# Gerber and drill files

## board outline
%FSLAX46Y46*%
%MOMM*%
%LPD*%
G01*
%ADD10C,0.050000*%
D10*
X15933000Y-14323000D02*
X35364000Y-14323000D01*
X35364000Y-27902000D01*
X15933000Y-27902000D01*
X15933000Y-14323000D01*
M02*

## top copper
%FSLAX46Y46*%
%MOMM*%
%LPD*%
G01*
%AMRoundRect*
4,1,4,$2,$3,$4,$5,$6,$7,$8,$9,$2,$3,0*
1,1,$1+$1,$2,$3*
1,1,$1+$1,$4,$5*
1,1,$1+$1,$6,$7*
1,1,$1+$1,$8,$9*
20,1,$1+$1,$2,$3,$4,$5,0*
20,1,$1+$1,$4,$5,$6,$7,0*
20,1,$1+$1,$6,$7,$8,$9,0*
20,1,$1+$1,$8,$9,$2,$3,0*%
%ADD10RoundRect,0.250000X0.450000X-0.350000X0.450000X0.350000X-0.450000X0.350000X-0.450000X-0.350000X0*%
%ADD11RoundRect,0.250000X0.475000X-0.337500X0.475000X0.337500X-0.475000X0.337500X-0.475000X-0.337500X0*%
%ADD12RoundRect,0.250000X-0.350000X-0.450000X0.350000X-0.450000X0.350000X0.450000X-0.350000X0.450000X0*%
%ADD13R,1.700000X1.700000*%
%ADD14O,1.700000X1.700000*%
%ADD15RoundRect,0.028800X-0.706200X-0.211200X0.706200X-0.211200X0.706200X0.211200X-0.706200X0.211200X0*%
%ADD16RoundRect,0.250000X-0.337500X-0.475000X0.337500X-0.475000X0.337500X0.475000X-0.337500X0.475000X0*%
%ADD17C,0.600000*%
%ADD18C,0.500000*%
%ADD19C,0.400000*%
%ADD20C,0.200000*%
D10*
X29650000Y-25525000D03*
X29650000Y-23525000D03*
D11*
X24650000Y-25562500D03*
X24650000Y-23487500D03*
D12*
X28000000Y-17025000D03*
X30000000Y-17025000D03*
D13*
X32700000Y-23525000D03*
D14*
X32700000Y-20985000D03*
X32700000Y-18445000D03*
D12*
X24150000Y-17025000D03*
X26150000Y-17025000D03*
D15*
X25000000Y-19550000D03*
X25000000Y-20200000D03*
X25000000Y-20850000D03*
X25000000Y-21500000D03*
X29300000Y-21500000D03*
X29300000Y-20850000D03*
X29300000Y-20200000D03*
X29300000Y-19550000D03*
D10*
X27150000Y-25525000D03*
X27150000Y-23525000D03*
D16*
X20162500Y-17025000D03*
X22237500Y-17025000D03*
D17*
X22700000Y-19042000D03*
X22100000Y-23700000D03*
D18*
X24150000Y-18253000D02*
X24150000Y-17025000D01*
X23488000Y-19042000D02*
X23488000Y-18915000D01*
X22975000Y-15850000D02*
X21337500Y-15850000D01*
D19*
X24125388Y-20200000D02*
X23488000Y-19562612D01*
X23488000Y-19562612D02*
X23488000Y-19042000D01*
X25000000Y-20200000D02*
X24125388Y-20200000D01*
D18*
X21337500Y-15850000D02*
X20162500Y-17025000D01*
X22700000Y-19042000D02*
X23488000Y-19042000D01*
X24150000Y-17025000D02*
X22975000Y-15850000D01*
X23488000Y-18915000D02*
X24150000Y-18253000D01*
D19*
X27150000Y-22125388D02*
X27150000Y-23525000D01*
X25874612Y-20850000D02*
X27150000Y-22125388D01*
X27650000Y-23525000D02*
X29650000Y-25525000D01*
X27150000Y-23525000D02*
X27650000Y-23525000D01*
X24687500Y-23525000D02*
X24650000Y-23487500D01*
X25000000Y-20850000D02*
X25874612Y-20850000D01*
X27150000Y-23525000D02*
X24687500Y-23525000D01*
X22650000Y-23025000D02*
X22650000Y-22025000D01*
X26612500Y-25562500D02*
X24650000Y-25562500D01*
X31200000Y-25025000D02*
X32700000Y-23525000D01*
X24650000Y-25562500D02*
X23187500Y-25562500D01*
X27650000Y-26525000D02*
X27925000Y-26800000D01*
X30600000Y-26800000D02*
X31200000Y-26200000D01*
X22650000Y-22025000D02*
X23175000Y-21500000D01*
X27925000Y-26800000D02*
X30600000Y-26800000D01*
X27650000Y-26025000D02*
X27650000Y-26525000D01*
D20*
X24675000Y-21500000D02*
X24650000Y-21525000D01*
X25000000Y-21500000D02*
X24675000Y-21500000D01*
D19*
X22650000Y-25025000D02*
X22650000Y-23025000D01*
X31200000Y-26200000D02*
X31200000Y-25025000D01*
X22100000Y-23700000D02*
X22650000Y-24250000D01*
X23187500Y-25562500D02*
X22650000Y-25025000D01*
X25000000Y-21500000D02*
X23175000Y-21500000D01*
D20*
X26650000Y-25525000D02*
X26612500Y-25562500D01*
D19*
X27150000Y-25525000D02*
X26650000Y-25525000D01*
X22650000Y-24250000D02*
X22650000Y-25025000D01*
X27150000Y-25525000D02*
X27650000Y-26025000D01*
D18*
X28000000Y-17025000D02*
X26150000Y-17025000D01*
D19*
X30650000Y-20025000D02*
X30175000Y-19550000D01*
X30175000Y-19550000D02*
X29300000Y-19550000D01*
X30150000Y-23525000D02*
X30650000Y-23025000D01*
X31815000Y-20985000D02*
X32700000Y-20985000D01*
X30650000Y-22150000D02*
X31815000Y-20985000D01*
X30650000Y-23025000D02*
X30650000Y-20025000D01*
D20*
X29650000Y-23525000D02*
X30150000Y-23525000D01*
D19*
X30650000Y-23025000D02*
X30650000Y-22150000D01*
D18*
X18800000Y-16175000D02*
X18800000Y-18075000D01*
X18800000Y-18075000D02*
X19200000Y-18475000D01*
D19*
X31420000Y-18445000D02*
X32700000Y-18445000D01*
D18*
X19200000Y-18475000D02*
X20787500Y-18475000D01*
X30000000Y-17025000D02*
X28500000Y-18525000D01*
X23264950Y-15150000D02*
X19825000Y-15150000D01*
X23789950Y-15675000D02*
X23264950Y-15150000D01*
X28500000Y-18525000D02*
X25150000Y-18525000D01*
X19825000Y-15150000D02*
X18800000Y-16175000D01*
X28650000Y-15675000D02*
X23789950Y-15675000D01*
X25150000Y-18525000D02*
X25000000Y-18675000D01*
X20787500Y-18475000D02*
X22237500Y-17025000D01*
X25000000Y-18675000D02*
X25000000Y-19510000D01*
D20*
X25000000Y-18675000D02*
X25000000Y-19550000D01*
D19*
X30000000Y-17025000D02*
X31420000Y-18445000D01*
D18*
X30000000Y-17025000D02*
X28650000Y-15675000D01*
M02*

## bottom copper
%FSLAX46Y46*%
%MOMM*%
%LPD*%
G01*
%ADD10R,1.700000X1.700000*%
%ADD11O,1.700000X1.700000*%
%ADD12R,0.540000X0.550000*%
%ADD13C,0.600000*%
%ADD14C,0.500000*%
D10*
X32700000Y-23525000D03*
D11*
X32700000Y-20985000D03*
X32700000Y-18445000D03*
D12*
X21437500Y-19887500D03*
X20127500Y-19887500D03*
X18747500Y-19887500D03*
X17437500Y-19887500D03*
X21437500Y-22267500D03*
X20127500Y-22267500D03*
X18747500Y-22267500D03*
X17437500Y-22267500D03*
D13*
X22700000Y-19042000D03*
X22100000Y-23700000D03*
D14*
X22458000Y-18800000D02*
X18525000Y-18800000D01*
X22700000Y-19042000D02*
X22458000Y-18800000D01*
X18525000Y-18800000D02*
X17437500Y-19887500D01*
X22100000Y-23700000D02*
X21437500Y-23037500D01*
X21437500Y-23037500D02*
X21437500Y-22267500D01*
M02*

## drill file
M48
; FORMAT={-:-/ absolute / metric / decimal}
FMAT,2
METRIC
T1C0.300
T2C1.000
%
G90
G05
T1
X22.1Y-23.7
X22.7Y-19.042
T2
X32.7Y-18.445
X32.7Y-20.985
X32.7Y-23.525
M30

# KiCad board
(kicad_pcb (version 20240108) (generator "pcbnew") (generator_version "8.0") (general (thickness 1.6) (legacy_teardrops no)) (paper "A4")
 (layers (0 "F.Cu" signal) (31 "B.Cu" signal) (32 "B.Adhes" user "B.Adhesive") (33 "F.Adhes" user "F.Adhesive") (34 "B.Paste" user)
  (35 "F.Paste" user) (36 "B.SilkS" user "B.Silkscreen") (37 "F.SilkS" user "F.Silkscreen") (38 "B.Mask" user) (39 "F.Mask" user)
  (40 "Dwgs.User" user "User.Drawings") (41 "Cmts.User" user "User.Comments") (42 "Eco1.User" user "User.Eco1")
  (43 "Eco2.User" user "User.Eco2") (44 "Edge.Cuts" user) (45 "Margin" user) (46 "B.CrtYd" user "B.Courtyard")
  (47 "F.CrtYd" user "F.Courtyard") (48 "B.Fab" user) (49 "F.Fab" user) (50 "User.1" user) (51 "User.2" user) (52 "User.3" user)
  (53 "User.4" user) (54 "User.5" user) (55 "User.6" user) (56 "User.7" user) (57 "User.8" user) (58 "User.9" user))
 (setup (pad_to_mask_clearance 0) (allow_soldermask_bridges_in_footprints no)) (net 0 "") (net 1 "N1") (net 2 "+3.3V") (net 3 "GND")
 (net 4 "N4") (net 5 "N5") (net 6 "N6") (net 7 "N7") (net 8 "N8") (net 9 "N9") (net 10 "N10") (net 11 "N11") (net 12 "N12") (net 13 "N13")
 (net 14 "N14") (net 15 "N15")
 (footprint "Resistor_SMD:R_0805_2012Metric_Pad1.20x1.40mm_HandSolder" (layer "F.Cu") (at 29.65 24.525 90)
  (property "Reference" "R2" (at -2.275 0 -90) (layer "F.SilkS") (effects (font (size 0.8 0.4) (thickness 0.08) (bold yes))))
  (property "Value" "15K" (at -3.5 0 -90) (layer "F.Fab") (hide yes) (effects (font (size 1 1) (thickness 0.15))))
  (pad "1" smd roundrect (at -1 0 90) (size 1.2 1.4) (layers "F.Cu" "F.Paste" "F.Mask") (roundrect_rratio 0.208333) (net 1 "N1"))
  (pad "2" smd roundrect (at 1 0 90) (size 1.2 1.4) (layers "F.Cu" "F.Paste" "F.Mask") (roundrect_rratio 0.208333) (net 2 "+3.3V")))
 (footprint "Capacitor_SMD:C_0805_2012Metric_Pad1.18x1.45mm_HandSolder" (layer "F.Cu") (at 24.65 24.525 90)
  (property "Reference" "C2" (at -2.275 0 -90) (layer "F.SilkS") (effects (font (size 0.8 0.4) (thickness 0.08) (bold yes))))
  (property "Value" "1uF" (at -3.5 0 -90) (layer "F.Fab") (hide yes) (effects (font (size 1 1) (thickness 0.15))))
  (pad "1" smd roundrect (at -1.0375 0 90) (size 1.175 1.45) (layers "F.Cu" "F.Paste" "F.Mask") (roundrect_rratio 0.212766) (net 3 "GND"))
  (pad "2" smd roundrect (at 1.0375 0 90) (size 1.175 1.45) (layers "F.Cu" "F.Paste" "F.Mask") (roundrect_rratio 0.212766) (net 1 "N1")))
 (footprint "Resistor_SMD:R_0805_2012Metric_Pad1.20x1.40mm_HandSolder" (layer "F.Cu") (at 29 17.025)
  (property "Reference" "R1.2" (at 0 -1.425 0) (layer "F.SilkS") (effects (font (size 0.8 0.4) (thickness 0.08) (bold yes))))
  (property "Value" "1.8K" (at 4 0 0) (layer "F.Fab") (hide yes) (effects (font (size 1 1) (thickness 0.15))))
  (pad "1" smd roundrect (at -1 0) (size 1.2 1.4) (layers "F.Cu" "F.Paste" "F.Mask") (roundrect_rratio 0.208333) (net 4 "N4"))
  (pad "2" smd roundrect (at 1 0) (size 1.2 1.4) (layers "F.Cu" "F.Paste" "F.Mask") (roundrect_rratio 0.208333) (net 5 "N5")))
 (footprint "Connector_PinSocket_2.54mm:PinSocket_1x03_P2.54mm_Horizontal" (layer "F.Cu") (at 32.7 23.525 180)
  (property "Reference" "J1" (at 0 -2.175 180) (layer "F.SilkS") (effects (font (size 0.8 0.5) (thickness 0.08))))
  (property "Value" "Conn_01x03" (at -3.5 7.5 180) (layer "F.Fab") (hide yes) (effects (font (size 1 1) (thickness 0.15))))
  (pad "1" thru_hole rect (at 0 0 180) (size 1.7 1.7) (drill 1) (layers "*.Cu" "*.Mask") (remove_unused_layers no) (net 3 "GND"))
  (pad "2" thru_hole oval (at 0 2.54 180) (size 1.7 1.7) (drill 1) (layers "*.Cu" "*.Mask") (remove_unused_layers no) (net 2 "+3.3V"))
  (pad "3" thru_hole oval (at 0 5.08 180) (size 1.7 1.7) (drill 1) (layers "*.Cu" "*.Mask") (remove_unused_layers no) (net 5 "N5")))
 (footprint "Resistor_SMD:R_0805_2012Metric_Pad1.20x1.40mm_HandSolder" (layer "F.Cu") (at 25.15 17.025)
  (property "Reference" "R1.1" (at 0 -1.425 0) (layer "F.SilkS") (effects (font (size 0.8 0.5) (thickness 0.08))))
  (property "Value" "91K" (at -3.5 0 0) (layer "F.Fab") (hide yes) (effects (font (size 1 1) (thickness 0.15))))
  (pad "1" smd roundrect (at -1 0) (size 1.2 1.4) (layers "F.Cu" "F.Paste" "F.Mask") (roundrect_rratio 0.208333) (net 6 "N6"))
  (pad "2" smd roundrect (at 1 0) (size 1.2 1.4) (layers "F.Cu" "F.Paste" "F.Mask") (roundrect_rratio 0.208333) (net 4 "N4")))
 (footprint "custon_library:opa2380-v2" (layer "F.Cu") (at 27.15 20.525)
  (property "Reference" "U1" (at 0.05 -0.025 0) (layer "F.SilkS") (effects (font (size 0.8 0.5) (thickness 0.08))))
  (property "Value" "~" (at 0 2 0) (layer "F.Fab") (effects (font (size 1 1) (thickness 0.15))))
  (pad "1" smd roundrect (at -2.15 -0.975) (size 1.47 0.48) (layers "F.Cu" "F.Paste" "F.Mask") (roundrect_rratio 0.06) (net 5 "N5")
   (solder_mask_margin 0.05))
  (pad "2" smd roundrect (at -2.15 -0.325) (size 1.47 0.48) (layers "F.Cu" "F.Paste" "F.Mask") (roundrect_rratio 0.06) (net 6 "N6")
   (solder_mask_margin 0.05))
  (pad "3" smd roundrect (at -2.15 0.325) (size 1.47 0.48) (layers "F.Cu" "F.Paste" "F.Mask") (roundrect_rratio 0.06) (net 1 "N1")
   (solder_mask_margin 0.05))
  (pad "4" smd roundrect (at -2.15 0.975) (size 1.47 0.48) (layers "F.Cu" "F.Paste" "F.Mask") (roundrect_rratio 0.06) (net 3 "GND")
   (solder_mask_margin 0.05))
  (pad "5" smd roundrect (at 2.15 0.975) (size 1.47 0.48) (layers "F.Cu" "F.Paste" "F.Mask") (roundrect_rratio 0.06) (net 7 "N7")
   (solder_mask_margin 0.05))
  (pad "6" smd roundrect (at 2.15 0.325) (size 1.47 0.48) (layers "F.Cu" "F.Paste" "F.Mask") (roundrect_rratio 0.06) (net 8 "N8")
   (solder_mask_margin 0.05))
  (pad "7" smd roundrect (at 2.15 -0.325) (size 1.47 0.48) (layers "F.Cu" "F.Paste" "F.Mask") (roundrect_rratio 0.06) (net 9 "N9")
   (solder_mask_margin 0.05))
  (pad "8" smd roundrect (at 2.15 -0.975) (size 1.47 0.48) (layers "F.Cu" "F.Paste" "F.Mask") (roundrect_rratio 0.06) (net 2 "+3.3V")
   (solder_mask_margin 0.05)))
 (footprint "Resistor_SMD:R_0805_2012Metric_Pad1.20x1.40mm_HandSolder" (layer "F.Cu") (at 27.15 24.525 90)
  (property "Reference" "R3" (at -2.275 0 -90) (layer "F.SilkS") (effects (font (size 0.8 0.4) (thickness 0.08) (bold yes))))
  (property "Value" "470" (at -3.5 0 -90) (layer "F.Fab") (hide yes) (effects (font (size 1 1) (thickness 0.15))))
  (pad "1" smd roundrect (at -1 0 90) (size 1.2 1.4) (layers "F.Cu" "F.Paste" "F.Mask") (roundrect_rratio 0.208333) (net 3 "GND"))
  (pad "2" smd roundrect (at 1 0 90) (size 1.2 1.4) (layers "F.Cu" "F.Paste" "F.Mask") (roundrect_rratio 0.208333) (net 1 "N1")))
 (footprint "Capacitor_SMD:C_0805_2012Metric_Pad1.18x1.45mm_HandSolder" (layer "F.Cu") (at 21.2 17.025)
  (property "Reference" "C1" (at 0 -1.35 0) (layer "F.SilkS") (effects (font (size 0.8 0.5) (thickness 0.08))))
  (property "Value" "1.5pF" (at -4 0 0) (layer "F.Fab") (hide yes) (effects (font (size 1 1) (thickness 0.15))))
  (pad "1" smd roundrect (at -1.0375 0) (size 1.175 1.45) (layers "F.Cu" "F.Paste" "F.Mask") (roundrect_rratio 0.212766) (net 6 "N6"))
  (pad "2" smd roundrect (at 1.0375 0) (size 1.175 1.45) (layers "F.Cu" "F.Paste" "F.Mask") (roundrect_rratio 0.212766) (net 5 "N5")))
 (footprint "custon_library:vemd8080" (layer "B.Cu") (at 19.4475 17.1675 180)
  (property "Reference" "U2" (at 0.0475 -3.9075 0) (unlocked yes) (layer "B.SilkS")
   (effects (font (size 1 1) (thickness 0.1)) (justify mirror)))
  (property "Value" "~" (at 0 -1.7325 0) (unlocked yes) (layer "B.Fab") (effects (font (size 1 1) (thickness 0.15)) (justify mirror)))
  (pad "1" smd rect (at -1.99 -2.72 180) (size 0.54 0.55) (layers "B.Cu" "B.Paste" "B.Mask") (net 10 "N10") (solder_mask_margin 0.05)
   (thermal_bridge_angle 45))
  (pad "2" smd rect (at -0.68 -2.72 180) (size 0.54 0.55) (layers "B.Cu" "B.Paste" "B.Mask") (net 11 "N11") (solder_mask_margin 0.05)
   (thermal_bridge_angle 45))
  (pad "3" smd rect (at 0.7 -2.72 180) (size 0.54 0.55) (layers "B.Cu" "B.Paste" "B.Mask") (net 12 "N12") (solder_mask_margin 0.05)
   (thermal_bridge_angle 45))
  (pad "4" smd rect (at 2.01 -2.72 180) (size 0.54 0.55) (layers "B.Cu" "B.Paste" "B.Mask") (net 6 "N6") (solder_mask_margin 0.05)
   (thermal_bridge_angle 45))
  (pad "5" smd rect (at -1.99 -5.1 180) (size 0.54 0.55) (layers "B.Cu" "B.Paste" "B.Mask") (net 3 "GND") (solder_mask_margin 0.05)
   (thermal_bridge_angle 45))
  (pad "6" smd rect (at -0.68 -5.1 180) (size 0.54 0.55) (layers "B.Cu" "B.Paste" "B.Mask") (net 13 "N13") (solder_mask_margin 0.05)
   (thermal_bridge_angle 45))
  (pad "7" smd rect (at 0.7 -5.1 180) (size 0.54 0.55) (layers "B.Cu" "B.Paste" "B.Mask") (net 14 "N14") (solder_mask_margin 0.05)
   (thermal_bridge_angle 45))
  (pad "8" smd rect (at 2.01 -5.1 180) (size 0.54 0.55) (layers "B.Cu" "B.Paste" "B.Mask") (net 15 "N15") (solder_mask_margin 0.05)
   (thermal_bridge_angle 45)))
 (gr_rect (start 15.933 14.323) (end 35.364 27.902) (stroke (width 0.05) (type default)) (fill none) (layer "Edge.Cuts"))
 (segment (start 24.15 18.253) (end 24.15 17.025) (width 0.5) (layer "F.Cu") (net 6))
 (segment (start 23.488 19.042) (end 23.488 18.915) (width 0.5) (layer "F.Cu") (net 6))
 (segment (start 22.975 15.85) (end 21.3375 15.85) (width 0.5) (layer "F.Cu") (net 6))
 (segment (start 24.125388 20.2) (end 23.488 19.562612) (width 0.4) (layer "F.Cu") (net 6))
 (segment (start 23.488 19.562612) (end 23.488 19.042) (width 0.4) (layer "F.Cu") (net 6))
 (segment (start 25 20.2) (end 24.125388 20.2) (width 0.4) (layer "F.Cu") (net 6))
 (segment (start 21.3375 15.85) (end 20.1625 17.025) (width 0.5) (layer "F.Cu") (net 6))
 (segment (start 22.7 19.042) (end 23.488 19.042) (width 0.5) (layer "F.Cu") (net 6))
 (segment (start 24.15 17.025) (end 22.975 15.85) (width 0.5) (layer "F.Cu") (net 6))
 (segment (start 23.488 18.915) (end 24.15 18.253) (width 0.5) (layer "F.Cu") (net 6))
 (via (at 22.7 19.042) (size 0.6) (drill 0.3) (layers "F.Cu" "B.Cu") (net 6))
 (segment (start 22.458 18.8) (end 18.525 18.8) (width 0.5) (layer "B.Cu") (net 6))
 (segment (start 22.7 19.042) (end 22.458 18.8) (width 0.5) (layer "B.Cu") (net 6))
 (segment (start 18.525 18.8) (end 17.4375 19.8875) (width 0.5) (layer "B.Cu") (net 6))
 (segment (start 27.15 22.125388) (end 27.15 23.525) (width 0.4) (layer "F.Cu") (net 1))
 (segment (start 25.874612 20.85) (end 27.15 22.125388) (width 0.4) (layer "F.Cu") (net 1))
 (segment (start 27.65 23.525) (end 29.65 25.525) (width 0.4) (layer "F.Cu") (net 1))
 (segment (start 27.15 23.525) (end 27.65 23.525) (width 0.4) (layer "F.Cu") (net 1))
 (segment (start 24.6875 23.525) (end 24.65 23.4875) (width 0.4) (layer "F.Cu") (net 1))
 (segment (start 25 20.85) (end 25.874612 20.85) (width 0.4) (layer "F.Cu") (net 1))
 (segment (start 27.15 23.525) (end 24.6875 23.525) (width 0.4) (layer "F.Cu") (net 1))
 (segment (start 22.65 23.025) (end 22.65 22.025) (width 0.4) (layer "F.Cu") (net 3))
 (segment (start 26.6125 25.5625) (end 24.65 25.5625) (width 0.4) (layer "F.Cu") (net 3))
 (segment (start 31.2 25.025) (end 32.7 23.525) (width 0.4) (layer "F.Cu") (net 3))
 (segment (start 24.65 25.5625) (end 23.1875 25.5625) (width 0.4) (layer "F.Cu") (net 3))
 (segment (start 27.65 26.525) (end 27.925 26.8) (width 0.4) (layer "F.Cu") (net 3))
 (segment (start 30.6 26.8) (end 31.2 26.2) (width 0.4) (layer "F.Cu") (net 3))
 (segment (start 22.65 22.025) (end 23.175 21.5) (width 0.4) (layer "F.Cu") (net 3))
 (segment (start 27.925 26.8) (end 30.6 26.8) (width 0.4) (layer "F.Cu") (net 3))
 (segment (start 27.65 26.025) (end 27.65 26.525) (width 0.4) (layer "F.Cu") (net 3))
 (segment (start 24.675 21.5) (end 24.65 21.525) (width 0.2) (layer "F.Cu") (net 3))
 (segment (start 25 21.5) (end 24.675 21.5) (width 0.2) (layer "F.Cu") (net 3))
 (segment (start 22.65 25.025) (end 22.65 23.025) (width 0.4) (layer "F.Cu") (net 3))
 (segment (start 31.2 26.2) (end 31.2 25.025) (width 0.4) (layer "F.Cu") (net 3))
 (segment (start 22.1 23.7) (end 22.65 24.25) (width 0.4) (layer "F.Cu") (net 3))
 (segment (start 23.1875 25.5625) (end 22.65 25.025) (width 0.4) (layer "F.Cu") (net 3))
 (segment (start 25 21.5) (end 23.175 21.5) (width 0.4) (layer "F.Cu") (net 3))
 (segment (start 26.65 25.525) (end 26.6125 25.5625) (width 0.2) (layer "F.Cu") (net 3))
 (segment (start 27.15 25.525) (end 26.65 25.525) (width 0.4) (layer "F.Cu") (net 3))
 (segment (start 22.65 24.25) (end 22.65 25.025) (width 0.4) (layer "F.Cu") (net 3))
 (segment (start 27.15 25.525) (end 27.65 26.025) (width 0.4) (layer "F.Cu") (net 3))
 (via (at 22.1 23.7) (size 0.6) (drill 0.3) (layers "F.Cu" "B.Cu") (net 3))
 (segment (start 22.1 23.7) (end 21.4375 23.0375) (width 0.5) (layer "B.Cu") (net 3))
 (segment (start 21.4375 23.0375) (end 21.4375 22.2675) (width 0.5) (layer "B.Cu") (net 3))
 (segment (start 28 17.025) (end 26.15 17.025) (width 0.5) (layer "F.Cu") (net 4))
 (segment (start 30.65 20.025) (end 30.175 19.55) (width 0.4) (layer "F.Cu") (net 2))
 (segment (start 30.175 19.55) (end 29.3 19.55) (width 0.4) (layer "F.Cu") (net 2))
 (segment (start 30.15 23.525) (end 30.65 23.025) (width 0.4) (layer "F.Cu") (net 2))
 (segment (start 31.815 20.985) (end 32.7 20.985) (width 0.4) (layer "F.Cu") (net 2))
 (segment (start 30.65 22.15) (end 31.815 20.985) (width 0.4) (layer "F.Cu") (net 2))
 (segment (start 30.65 23.025) (end 30.65 20.025) (width 0.4) (layer "F.Cu") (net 2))
 (segment (start 29.65 23.525) (end 30.15 23.525) (width 0.2) (layer "F.Cu") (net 2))
 (segment (start 30.65 23.025) (end 30.65 22.15) (width 0.4) (layer "F.Cu") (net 2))
 (segment (start 18.8 16.175) (end 18.8 18.075) (width 0.5) (layer "F.Cu") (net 5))
 (segment (start 18.8 18.075) (end 19.2 18.475) (width 0.5) (layer "F.Cu") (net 5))
 (segment (start 31.42 18.445) (end 32.7 18.445) (width 0.4) (layer "F.Cu") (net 5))
 (segment (start 19.2 18.475) (end 20.7875 18.475) (width 0.5) (layer "F.Cu") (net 5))
 (segment (start 30 17.025) (end 28.5 18.525) (width 0.5) (layer "F.Cu") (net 5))
 (segment (start 23.26495 15.15) (end 19.825 15.15) (width 0.5) (layer "F.Cu") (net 5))
 (segment (start 23.78995 15.675) (end 23.26495 15.15) (width 0.5) (layer "F.Cu") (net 5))
 (segment (start 28.5 18.525) (end 25.15 18.525) (width 0.5) (layer "F.Cu") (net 5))
 (segment (start 19.825 15.15) (end 18.8 16.175) (width 0.5) (layer "F.Cu") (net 5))
 (segment (start 28.65 15.675) (end 23.78995 15.675) (width 0.5) (layer "F.Cu") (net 5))
 (segment (start 25.15 18.525) (end 25 18.675) (width 0.5) (layer "F.Cu") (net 5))
 (segment (start 20.7875 18.475) (end 22.2375 17.025) (width 0.5) (layer "F.Cu") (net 5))
 (segment (start 25 18.675) (end 25 19.51) (width 0.5) (layer "F.Cu") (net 5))
 (segment (start 25 18.675) (end 25 19.55) (width 0.2) (layer "F.Cu") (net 5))
 (segment (start 30 17.025) (end 31.42 18.445) (width 0.4) (layer "F.Cu") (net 5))
 (segment (start 30 17.025) (end 28.65 15.675) (width 0.5) (layer "F.Cu") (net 5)))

